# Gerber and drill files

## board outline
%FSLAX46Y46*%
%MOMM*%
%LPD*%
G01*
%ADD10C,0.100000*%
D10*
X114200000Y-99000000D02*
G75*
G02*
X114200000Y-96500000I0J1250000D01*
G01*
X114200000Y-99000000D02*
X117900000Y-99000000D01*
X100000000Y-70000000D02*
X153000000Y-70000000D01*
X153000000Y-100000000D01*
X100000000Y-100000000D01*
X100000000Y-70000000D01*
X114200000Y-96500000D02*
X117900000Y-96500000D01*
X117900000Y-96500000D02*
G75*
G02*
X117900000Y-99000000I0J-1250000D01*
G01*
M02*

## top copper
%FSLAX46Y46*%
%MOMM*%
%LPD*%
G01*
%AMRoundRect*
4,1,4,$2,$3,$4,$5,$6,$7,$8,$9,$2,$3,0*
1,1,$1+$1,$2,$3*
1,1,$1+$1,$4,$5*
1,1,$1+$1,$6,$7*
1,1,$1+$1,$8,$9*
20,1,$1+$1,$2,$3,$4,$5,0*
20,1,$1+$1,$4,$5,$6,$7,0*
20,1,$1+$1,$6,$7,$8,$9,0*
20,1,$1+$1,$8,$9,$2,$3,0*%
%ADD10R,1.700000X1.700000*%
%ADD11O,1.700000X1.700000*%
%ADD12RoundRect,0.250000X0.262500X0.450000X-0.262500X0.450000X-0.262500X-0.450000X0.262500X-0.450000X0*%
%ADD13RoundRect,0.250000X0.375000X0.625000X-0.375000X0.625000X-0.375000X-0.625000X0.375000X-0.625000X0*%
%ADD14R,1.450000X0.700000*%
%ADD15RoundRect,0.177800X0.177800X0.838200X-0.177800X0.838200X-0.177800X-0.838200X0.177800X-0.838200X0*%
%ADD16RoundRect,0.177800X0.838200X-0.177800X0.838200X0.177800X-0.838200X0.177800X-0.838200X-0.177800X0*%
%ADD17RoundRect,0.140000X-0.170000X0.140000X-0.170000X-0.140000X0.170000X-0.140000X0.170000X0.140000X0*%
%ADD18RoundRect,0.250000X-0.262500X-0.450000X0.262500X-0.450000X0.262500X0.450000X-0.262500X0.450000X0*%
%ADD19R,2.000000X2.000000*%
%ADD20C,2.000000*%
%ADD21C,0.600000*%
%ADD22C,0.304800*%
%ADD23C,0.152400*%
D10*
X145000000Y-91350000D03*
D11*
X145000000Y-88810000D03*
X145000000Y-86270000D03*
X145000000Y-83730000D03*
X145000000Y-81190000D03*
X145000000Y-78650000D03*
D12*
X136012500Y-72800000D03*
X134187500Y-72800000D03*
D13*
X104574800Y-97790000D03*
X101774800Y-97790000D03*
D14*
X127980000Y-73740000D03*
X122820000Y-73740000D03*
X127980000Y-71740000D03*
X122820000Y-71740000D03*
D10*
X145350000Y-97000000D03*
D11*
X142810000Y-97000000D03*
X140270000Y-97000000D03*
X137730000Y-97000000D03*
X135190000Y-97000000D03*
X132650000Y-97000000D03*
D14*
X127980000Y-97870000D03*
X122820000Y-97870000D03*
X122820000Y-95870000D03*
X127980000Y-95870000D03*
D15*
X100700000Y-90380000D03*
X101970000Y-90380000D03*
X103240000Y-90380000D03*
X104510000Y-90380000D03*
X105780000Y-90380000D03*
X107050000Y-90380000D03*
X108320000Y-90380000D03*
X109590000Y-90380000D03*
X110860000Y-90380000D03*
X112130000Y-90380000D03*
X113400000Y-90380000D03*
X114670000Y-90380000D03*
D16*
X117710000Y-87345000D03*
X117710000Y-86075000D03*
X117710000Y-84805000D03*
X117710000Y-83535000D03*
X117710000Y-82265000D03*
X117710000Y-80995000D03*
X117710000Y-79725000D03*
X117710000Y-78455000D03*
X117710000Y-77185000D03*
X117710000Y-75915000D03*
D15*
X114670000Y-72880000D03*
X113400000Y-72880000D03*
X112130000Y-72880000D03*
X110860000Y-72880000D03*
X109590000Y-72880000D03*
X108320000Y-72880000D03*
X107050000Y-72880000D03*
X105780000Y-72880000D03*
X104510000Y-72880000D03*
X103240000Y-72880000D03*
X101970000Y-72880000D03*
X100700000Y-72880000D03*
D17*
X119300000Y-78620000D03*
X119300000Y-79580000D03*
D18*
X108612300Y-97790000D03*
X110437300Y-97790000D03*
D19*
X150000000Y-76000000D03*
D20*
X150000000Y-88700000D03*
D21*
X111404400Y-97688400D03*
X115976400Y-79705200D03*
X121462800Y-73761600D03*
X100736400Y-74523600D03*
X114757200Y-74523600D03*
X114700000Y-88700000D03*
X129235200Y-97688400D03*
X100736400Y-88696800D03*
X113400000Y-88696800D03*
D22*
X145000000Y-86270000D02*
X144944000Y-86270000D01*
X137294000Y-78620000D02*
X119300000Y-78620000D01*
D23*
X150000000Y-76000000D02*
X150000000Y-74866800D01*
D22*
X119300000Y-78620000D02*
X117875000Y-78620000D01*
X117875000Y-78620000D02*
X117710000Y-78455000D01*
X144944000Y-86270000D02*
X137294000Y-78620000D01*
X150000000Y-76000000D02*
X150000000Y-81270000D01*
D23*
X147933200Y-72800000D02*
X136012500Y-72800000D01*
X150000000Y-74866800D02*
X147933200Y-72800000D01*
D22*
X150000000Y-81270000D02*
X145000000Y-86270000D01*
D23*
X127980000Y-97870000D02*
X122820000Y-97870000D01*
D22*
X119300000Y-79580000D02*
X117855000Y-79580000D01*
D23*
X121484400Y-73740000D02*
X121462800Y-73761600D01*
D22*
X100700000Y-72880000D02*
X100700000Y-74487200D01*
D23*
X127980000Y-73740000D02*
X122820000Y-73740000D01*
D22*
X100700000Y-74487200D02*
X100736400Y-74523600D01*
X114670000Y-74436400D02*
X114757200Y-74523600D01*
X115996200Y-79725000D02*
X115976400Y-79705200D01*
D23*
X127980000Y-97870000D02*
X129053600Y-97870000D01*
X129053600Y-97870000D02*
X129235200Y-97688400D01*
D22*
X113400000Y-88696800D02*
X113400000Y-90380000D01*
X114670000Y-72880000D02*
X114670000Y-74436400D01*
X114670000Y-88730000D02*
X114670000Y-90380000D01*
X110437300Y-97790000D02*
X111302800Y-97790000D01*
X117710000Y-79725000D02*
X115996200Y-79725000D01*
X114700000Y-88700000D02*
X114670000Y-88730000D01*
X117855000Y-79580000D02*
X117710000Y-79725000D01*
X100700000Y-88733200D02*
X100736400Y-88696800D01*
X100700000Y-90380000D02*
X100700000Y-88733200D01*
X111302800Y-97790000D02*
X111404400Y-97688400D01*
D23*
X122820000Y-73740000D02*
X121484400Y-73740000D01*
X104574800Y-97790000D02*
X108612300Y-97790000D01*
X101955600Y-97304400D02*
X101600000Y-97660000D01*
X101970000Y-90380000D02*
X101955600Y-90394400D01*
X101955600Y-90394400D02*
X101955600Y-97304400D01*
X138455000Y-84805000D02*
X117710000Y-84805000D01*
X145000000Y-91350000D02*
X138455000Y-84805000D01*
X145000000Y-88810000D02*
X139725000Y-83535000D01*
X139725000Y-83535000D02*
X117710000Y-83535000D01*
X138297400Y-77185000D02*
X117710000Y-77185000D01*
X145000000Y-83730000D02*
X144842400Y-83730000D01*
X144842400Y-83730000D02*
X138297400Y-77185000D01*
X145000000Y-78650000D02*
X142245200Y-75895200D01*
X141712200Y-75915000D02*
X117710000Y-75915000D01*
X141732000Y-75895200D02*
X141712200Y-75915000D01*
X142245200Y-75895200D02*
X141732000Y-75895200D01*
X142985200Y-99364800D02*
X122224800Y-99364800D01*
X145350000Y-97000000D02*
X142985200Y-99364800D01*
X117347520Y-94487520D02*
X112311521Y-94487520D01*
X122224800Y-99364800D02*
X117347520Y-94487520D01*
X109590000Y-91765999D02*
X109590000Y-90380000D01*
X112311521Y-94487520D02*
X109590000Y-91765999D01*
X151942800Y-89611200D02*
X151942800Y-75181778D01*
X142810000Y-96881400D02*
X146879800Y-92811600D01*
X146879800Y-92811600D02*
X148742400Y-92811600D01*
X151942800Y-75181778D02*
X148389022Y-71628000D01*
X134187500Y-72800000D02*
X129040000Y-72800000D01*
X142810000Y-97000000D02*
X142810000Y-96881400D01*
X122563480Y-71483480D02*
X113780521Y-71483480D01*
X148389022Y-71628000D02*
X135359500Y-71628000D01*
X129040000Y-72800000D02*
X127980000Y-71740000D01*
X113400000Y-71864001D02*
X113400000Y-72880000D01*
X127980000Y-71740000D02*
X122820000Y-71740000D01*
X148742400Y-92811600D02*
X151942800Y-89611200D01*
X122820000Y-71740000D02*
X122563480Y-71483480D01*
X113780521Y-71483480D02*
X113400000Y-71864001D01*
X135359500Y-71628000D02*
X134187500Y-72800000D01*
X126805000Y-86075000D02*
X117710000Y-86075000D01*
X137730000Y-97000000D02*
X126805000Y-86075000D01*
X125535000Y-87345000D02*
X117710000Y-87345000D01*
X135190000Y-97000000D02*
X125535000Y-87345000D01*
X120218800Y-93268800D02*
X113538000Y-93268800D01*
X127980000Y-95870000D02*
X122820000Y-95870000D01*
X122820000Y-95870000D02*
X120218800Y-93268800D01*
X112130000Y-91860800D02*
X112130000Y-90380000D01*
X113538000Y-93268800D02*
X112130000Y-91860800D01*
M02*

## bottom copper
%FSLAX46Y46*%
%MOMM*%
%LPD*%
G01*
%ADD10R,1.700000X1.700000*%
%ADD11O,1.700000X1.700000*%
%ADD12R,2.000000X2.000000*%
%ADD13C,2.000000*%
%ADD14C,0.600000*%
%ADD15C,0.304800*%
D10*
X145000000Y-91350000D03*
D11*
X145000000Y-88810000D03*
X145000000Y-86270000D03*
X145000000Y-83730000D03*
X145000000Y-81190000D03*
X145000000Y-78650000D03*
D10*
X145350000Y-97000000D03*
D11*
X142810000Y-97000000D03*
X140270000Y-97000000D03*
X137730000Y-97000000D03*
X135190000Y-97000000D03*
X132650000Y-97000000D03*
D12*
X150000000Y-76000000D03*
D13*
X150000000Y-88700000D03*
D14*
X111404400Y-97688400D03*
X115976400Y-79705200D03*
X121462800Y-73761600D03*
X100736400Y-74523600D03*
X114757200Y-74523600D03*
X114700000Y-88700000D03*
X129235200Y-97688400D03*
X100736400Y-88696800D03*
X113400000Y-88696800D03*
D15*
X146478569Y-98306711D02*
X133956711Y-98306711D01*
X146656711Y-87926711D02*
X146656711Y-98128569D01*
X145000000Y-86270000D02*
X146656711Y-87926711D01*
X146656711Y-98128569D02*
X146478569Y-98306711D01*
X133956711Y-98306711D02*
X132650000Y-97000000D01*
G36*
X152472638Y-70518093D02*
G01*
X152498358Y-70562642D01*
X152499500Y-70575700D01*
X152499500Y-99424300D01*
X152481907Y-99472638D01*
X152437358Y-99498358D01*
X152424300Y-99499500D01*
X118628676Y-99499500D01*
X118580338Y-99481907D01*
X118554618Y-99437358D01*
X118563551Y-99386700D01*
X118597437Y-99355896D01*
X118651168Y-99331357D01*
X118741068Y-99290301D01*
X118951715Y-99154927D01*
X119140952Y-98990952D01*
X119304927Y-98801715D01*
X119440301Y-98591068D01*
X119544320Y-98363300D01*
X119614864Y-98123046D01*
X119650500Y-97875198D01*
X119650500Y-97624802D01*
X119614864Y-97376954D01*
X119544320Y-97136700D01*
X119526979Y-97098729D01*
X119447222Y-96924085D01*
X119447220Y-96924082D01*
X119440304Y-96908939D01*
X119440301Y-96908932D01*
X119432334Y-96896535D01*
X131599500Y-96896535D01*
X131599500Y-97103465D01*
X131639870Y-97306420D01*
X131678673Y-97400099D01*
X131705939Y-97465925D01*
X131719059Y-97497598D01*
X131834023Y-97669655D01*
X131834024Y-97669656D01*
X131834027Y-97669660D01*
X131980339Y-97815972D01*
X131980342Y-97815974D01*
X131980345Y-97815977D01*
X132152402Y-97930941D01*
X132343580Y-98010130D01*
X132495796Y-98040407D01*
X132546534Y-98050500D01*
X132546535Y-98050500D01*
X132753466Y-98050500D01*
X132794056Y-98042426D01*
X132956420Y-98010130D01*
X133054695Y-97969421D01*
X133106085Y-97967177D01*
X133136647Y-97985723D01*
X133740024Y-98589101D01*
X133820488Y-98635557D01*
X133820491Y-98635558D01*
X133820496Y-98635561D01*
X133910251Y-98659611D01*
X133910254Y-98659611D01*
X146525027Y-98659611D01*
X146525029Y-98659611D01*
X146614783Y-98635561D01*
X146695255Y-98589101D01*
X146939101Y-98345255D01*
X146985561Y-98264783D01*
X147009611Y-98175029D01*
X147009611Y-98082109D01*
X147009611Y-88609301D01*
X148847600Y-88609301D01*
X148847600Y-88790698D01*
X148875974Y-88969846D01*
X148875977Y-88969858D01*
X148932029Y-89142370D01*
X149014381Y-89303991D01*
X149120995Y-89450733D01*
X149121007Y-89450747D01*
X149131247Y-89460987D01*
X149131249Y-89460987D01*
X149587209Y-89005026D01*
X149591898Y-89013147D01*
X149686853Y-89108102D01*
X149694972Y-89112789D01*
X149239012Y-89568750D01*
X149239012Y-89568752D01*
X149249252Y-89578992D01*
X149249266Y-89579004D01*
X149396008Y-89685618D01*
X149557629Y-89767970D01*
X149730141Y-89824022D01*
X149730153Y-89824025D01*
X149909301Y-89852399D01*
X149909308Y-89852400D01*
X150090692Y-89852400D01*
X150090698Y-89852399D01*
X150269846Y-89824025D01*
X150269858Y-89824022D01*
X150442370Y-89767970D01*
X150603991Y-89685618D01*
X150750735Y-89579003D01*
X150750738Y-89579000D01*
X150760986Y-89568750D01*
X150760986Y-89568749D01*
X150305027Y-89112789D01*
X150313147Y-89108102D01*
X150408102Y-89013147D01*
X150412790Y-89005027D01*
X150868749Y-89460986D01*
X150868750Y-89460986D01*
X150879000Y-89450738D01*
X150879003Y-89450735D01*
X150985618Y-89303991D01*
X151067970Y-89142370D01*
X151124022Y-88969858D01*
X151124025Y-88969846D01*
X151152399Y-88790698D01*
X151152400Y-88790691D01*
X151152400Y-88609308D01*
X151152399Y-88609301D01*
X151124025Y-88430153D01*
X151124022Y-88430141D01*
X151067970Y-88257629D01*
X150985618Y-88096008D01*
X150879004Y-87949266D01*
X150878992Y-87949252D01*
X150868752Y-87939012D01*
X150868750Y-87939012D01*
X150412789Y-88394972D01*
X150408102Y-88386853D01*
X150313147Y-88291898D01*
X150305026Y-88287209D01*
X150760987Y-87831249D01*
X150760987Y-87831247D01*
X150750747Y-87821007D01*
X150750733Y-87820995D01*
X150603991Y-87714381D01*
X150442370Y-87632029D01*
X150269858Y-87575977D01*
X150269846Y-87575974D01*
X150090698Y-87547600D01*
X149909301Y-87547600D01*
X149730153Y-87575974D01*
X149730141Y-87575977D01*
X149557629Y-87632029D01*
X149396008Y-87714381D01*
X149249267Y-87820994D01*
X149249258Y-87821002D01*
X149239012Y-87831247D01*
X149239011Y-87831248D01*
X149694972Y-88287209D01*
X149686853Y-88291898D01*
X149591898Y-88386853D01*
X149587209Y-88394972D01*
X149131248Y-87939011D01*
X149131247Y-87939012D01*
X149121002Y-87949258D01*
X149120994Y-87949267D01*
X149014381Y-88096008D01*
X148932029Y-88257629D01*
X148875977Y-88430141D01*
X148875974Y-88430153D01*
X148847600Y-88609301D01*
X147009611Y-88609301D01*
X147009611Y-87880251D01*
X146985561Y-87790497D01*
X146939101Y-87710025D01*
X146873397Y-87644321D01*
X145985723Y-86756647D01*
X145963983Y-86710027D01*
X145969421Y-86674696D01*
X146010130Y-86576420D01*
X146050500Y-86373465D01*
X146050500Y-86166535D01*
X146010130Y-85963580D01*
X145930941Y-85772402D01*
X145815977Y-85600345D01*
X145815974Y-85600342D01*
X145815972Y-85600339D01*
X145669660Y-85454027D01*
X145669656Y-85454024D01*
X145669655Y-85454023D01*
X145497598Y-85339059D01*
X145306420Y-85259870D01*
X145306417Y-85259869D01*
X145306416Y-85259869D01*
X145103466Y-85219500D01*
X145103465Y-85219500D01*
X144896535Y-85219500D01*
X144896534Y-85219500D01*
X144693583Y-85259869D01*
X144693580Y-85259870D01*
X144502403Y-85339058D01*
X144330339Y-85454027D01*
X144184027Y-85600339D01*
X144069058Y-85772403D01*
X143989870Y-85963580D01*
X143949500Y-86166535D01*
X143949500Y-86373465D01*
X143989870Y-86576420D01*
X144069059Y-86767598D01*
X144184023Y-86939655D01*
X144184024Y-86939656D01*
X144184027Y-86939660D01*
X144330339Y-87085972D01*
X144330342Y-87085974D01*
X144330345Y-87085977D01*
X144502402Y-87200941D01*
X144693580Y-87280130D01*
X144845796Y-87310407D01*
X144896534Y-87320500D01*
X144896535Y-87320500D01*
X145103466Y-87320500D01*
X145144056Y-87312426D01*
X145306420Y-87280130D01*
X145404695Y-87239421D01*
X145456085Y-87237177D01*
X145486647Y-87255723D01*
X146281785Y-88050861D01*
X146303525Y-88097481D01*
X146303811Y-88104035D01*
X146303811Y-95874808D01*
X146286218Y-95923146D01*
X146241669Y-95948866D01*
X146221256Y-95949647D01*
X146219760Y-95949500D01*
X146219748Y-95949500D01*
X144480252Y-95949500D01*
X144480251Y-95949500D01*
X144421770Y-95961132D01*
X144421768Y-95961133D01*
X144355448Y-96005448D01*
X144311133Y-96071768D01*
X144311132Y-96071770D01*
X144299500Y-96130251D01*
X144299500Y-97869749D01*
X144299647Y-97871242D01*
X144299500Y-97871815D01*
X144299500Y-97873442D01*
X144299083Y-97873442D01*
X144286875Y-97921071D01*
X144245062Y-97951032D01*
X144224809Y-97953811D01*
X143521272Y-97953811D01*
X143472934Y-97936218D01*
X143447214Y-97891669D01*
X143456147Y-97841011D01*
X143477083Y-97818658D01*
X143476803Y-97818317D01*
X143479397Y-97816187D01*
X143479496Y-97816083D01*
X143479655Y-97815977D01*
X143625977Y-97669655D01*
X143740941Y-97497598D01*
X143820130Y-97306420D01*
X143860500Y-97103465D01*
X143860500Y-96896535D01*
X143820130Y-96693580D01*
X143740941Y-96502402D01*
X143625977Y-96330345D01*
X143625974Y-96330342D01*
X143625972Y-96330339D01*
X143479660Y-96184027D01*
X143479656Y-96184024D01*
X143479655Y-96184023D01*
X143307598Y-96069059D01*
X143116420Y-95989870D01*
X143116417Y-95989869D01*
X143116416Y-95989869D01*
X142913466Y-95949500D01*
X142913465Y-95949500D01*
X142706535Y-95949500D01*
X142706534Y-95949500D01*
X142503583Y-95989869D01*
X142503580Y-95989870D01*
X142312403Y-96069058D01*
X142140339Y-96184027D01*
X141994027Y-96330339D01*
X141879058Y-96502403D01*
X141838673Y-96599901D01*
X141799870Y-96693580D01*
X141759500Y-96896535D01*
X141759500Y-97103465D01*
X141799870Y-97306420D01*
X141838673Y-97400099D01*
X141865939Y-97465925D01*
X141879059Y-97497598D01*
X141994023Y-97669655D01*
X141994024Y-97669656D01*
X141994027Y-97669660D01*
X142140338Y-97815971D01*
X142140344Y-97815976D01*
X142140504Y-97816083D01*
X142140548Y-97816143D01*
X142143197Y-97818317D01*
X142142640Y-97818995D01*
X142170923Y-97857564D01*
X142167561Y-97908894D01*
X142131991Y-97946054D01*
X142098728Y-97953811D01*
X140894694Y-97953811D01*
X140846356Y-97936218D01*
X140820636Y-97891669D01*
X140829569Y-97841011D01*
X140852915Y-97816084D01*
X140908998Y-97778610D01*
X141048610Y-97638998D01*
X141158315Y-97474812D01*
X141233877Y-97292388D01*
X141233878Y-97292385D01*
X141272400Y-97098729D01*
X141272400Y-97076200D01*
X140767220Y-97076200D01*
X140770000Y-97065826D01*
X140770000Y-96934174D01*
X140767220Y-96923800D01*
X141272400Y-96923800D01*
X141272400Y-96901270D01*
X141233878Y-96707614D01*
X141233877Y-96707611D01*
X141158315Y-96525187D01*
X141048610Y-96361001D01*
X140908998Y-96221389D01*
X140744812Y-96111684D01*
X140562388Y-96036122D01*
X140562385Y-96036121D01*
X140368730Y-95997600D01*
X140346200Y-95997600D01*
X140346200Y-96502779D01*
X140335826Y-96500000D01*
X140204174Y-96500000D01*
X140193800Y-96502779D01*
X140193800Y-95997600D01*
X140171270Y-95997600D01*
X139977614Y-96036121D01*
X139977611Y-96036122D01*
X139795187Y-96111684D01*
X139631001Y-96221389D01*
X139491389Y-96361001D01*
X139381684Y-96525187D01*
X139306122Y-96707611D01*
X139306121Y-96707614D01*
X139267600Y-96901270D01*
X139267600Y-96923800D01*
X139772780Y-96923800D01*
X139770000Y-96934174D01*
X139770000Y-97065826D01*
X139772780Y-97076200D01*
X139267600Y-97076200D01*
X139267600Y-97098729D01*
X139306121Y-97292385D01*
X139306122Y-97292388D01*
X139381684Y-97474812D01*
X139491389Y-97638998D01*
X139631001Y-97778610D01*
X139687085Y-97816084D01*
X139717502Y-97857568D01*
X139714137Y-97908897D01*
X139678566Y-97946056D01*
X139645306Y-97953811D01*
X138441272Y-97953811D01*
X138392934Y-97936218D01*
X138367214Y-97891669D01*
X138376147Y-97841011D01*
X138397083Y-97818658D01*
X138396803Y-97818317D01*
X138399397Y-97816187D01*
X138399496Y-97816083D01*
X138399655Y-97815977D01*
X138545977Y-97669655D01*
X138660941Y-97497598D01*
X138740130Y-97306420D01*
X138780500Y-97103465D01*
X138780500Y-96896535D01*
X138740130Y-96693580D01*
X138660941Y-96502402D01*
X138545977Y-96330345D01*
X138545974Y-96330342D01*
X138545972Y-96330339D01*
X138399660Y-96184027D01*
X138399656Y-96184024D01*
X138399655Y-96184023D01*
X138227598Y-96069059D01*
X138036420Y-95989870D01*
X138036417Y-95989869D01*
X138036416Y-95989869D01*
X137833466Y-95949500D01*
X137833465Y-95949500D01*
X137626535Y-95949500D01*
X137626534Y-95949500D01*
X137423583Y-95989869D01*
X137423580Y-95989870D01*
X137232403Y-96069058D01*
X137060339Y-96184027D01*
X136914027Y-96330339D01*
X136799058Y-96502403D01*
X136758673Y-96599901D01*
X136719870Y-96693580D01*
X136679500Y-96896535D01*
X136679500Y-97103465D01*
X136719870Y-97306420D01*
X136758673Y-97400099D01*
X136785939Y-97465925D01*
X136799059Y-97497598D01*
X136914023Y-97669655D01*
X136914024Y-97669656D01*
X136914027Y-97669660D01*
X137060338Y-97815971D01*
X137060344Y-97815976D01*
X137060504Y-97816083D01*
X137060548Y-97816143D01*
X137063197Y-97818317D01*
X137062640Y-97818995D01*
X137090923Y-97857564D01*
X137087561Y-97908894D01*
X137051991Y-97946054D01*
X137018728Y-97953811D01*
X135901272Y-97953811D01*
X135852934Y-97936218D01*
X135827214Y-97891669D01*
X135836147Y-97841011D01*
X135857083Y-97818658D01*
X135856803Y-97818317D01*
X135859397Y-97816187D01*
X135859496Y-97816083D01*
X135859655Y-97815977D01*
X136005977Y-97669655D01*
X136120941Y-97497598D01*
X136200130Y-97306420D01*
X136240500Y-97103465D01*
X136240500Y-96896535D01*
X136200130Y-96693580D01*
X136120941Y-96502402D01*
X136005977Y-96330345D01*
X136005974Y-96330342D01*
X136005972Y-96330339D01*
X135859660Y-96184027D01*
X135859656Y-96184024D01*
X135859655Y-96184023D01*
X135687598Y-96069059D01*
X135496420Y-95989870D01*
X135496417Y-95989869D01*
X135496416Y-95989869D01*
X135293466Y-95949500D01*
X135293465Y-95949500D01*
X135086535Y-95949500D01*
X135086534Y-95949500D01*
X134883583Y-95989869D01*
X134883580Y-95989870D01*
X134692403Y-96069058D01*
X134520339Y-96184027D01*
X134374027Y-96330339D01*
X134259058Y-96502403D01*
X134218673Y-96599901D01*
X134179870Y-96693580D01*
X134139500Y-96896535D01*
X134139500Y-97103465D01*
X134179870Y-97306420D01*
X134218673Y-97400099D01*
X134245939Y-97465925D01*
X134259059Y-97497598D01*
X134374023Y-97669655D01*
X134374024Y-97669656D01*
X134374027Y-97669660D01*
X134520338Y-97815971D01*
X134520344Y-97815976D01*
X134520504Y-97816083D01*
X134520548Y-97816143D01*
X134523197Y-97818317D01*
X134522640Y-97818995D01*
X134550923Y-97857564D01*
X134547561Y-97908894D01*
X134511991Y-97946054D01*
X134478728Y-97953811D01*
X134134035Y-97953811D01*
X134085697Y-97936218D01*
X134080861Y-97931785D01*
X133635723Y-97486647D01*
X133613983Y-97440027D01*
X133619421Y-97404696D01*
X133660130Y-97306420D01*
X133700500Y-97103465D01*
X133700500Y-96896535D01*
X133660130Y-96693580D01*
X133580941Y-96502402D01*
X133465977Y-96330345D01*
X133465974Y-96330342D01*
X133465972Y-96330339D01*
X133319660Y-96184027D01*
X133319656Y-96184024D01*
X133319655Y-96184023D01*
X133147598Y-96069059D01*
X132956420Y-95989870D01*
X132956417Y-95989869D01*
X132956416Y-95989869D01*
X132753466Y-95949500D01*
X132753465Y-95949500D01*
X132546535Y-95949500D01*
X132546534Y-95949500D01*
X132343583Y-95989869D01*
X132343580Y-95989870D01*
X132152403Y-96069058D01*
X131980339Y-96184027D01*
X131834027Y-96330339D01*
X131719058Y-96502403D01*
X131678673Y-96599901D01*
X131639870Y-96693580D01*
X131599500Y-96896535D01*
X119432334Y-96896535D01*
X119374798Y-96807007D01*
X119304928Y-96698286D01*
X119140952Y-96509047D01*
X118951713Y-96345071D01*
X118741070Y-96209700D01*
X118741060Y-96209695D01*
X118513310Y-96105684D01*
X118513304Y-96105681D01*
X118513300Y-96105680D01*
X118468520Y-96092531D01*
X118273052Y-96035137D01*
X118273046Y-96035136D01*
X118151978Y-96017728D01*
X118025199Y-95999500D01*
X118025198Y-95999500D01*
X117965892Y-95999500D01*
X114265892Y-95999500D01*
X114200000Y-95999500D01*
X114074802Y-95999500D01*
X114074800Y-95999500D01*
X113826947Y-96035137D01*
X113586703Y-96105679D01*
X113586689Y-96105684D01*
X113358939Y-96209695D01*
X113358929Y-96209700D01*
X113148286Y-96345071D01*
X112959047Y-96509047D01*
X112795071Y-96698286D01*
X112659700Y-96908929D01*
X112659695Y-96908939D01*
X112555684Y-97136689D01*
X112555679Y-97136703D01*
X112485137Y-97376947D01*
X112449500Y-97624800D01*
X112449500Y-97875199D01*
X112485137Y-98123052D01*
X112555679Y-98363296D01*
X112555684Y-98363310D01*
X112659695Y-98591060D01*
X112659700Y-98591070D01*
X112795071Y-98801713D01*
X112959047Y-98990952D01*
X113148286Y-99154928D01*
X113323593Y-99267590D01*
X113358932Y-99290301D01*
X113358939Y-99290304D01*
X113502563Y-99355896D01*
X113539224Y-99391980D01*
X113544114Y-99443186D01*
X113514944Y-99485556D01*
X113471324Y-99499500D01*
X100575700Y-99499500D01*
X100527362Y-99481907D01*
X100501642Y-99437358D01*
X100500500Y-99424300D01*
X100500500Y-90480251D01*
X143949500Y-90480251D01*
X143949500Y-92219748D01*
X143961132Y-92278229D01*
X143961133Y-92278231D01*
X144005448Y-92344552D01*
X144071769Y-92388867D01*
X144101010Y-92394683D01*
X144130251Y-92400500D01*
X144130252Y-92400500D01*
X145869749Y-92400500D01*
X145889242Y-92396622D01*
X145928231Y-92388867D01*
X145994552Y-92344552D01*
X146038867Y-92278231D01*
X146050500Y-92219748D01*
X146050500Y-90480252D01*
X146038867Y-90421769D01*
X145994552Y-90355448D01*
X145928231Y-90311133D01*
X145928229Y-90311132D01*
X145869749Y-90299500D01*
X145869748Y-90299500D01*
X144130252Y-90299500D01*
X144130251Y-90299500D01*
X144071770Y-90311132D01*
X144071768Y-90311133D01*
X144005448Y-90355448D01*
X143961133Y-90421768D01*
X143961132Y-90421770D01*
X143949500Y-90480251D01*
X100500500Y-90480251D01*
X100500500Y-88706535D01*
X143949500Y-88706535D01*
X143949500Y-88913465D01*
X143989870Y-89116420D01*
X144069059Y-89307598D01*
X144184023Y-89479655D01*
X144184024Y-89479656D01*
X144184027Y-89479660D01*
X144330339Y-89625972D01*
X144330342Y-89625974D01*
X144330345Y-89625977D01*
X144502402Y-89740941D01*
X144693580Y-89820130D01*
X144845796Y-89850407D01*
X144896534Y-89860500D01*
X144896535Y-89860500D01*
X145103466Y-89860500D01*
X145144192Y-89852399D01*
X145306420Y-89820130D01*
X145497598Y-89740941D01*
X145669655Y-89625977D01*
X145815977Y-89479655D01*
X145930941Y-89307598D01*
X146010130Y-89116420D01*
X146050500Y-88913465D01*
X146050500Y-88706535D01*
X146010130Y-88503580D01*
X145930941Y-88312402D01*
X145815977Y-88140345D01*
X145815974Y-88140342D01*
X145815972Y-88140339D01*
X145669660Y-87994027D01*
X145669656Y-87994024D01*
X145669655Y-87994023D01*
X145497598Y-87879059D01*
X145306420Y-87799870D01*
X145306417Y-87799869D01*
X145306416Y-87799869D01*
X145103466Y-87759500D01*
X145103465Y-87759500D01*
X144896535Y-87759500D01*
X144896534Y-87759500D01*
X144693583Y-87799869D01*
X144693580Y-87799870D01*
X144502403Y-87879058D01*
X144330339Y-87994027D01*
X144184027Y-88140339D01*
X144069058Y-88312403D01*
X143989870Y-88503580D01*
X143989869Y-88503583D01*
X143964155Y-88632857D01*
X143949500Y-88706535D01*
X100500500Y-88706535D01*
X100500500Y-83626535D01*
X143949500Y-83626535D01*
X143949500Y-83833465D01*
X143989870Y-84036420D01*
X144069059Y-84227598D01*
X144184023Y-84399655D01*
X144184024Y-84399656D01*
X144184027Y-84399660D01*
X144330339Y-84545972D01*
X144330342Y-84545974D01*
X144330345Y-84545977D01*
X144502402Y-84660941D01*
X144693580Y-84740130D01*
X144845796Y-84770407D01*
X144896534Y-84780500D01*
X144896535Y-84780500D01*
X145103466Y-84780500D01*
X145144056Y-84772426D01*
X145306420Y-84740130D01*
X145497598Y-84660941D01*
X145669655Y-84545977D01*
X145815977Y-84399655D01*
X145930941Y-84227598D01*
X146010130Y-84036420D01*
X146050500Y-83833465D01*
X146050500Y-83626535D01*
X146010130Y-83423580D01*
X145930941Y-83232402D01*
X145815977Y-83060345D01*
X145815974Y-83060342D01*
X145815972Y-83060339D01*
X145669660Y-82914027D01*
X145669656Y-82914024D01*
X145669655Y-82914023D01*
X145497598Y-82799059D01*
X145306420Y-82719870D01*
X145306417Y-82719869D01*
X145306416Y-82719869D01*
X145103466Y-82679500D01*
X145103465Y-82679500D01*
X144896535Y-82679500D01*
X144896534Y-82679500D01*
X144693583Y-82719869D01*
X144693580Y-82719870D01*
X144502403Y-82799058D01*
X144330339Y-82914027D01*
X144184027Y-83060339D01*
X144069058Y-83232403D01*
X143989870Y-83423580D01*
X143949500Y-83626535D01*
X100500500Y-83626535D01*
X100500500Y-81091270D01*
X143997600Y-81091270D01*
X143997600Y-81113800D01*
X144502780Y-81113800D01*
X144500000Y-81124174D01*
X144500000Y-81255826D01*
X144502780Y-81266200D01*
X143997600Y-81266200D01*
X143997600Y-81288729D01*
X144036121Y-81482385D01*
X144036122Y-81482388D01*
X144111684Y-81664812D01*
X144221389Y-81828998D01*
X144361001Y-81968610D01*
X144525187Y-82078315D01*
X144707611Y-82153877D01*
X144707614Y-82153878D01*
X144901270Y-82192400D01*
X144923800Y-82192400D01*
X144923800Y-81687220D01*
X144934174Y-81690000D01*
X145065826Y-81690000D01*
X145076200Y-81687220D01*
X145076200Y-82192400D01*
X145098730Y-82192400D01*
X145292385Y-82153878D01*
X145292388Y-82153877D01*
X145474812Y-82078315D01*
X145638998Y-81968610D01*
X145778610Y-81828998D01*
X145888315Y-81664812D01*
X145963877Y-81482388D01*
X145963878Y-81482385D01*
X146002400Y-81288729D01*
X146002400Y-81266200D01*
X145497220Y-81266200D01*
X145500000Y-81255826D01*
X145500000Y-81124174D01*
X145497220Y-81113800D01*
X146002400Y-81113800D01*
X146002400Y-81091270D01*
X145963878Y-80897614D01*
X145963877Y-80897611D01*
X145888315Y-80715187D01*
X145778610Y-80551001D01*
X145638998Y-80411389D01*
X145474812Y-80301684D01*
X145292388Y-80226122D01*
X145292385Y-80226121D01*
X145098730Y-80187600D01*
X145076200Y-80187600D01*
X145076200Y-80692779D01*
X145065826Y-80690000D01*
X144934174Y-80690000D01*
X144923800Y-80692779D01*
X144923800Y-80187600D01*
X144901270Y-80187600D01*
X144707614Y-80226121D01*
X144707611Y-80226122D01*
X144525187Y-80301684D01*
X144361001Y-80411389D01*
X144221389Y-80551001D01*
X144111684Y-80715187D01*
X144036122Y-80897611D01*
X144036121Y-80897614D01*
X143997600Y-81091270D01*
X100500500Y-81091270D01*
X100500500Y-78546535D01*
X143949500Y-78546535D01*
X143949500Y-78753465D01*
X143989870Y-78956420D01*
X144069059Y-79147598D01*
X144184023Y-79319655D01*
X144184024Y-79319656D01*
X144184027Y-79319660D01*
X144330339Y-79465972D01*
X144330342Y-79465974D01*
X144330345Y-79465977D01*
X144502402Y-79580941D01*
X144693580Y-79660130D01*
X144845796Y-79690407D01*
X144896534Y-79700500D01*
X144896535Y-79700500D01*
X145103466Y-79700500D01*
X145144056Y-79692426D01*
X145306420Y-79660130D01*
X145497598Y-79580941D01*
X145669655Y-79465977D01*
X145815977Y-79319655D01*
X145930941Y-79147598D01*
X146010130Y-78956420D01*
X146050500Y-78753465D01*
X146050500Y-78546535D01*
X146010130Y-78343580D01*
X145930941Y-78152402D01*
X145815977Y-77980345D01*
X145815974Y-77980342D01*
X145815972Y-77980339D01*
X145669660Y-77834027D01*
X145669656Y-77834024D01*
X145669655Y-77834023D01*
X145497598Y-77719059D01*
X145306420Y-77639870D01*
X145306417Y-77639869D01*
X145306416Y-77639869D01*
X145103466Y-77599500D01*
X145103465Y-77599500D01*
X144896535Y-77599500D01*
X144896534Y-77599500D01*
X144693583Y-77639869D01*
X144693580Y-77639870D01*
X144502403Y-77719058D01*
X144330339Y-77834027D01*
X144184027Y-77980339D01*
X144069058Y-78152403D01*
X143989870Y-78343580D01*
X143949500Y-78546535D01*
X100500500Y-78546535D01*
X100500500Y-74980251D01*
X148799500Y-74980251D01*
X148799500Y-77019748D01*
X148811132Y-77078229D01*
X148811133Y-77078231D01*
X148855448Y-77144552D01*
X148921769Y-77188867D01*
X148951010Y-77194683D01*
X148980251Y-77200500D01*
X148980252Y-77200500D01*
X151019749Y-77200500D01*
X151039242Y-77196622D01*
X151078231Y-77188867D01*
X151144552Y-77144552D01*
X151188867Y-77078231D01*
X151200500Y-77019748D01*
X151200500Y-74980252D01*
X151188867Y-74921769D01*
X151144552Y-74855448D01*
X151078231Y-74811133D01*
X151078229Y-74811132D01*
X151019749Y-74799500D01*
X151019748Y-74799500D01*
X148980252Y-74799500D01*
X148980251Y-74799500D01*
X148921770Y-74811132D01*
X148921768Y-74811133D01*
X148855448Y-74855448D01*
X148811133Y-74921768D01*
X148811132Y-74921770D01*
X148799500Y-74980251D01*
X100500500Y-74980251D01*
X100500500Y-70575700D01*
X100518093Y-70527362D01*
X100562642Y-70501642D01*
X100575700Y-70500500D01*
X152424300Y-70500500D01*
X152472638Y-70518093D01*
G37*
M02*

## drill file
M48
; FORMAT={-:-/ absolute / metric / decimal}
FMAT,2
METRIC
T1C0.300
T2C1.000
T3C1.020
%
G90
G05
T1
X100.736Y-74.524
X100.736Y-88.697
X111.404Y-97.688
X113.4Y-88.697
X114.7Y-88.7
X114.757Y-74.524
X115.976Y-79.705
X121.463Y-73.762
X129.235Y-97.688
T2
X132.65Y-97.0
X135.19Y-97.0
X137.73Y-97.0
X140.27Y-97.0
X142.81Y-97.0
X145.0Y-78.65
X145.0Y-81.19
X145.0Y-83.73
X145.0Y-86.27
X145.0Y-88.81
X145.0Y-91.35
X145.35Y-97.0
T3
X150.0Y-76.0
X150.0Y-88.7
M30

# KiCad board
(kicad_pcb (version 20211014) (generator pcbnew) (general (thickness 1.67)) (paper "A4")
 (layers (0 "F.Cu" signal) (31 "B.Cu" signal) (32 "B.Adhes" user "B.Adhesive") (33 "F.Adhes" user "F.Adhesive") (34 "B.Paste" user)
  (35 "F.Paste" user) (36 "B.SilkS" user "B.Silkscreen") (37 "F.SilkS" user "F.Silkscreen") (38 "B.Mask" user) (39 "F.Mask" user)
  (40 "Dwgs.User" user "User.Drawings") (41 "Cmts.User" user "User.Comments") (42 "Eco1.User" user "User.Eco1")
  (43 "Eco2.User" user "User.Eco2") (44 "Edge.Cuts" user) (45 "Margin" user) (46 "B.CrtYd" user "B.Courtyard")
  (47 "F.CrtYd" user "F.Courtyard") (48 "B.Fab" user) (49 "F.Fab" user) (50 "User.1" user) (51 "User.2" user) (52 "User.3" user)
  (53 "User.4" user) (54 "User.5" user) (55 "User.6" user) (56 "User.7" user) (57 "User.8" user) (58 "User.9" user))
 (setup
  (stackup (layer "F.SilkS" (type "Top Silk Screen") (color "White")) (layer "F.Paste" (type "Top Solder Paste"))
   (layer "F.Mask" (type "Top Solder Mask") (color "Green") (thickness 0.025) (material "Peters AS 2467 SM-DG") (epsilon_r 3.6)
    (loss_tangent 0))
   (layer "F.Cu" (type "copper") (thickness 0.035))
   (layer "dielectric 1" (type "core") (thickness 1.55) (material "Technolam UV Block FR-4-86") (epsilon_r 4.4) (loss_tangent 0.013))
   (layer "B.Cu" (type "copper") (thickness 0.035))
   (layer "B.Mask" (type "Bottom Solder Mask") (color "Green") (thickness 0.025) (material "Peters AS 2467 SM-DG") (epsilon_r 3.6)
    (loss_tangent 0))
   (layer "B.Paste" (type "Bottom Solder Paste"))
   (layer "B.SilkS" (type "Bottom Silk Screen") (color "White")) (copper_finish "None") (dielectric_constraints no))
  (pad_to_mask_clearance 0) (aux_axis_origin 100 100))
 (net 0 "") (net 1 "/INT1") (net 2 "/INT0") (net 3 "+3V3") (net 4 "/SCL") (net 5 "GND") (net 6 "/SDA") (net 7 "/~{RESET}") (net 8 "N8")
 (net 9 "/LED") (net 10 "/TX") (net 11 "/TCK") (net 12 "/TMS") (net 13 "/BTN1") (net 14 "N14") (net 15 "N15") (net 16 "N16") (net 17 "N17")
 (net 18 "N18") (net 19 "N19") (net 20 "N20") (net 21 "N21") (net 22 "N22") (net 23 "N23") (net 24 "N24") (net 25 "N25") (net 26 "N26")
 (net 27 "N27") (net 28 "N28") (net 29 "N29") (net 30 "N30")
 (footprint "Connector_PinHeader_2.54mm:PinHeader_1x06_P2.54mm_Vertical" (layer "F.Cu") (at 145 91.35 180)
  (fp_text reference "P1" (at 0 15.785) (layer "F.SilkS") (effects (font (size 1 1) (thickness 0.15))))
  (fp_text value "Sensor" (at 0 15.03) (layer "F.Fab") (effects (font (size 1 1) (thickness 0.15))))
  (pad "1" thru_hole rect locked (at 0 0 180) (size 1.7 1.7) (drill 1) (layers *.Cu *.Mask) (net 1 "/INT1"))
  (pad "2" thru_hole oval locked (at 0 2.54 180) (size 1.7 1.7) (drill 1) (layers *.Cu *.Mask) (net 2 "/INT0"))
  (pad "3" thru_hole oval locked (at 0 5.08 180) (size 1.7 1.7) (drill 1) (layers *.Cu *.Mask) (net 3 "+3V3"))
  (pad "4" thru_hole oval locked (at 0 7.62 180) (size 1.7 1.7) (drill 1) (layers *.Cu *.Mask) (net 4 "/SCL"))
  (pad "5" thru_hole oval locked (at 0 10.16 180) (size 1.7 1.7) (drill 1) (layers *.Cu *.Mask) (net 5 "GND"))
  (pad "6" thru_hole oval locked (at 0 12.7 180) (size 1.7 1.7) (drill 1) (layers *.Cu *.Mask) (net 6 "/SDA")))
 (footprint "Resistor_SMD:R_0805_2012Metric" (layer "F.Cu") (at 135.1 72.8 180)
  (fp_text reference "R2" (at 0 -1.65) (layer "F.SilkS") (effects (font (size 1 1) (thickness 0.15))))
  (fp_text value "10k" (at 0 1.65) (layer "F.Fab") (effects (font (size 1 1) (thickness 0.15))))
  (pad "1" smd roundrect locked (at -0.9125 0 180) (size 1.025 1.4) (layers "F.Cu" "F.Paste" "F.Mask") (roundrect_rratio 0.243902439)
   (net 3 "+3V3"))
  (pad "2" smd roundrect locked (at 0.9125 0 180) (size 1.025 1.4) (layers "F.Cu" "F.Paste" "F.Mask") (roundrect_rratio 0.243902439)
   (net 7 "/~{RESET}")))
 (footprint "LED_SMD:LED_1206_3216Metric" (layer "F.Cu") (at 103.1748 97.79 180)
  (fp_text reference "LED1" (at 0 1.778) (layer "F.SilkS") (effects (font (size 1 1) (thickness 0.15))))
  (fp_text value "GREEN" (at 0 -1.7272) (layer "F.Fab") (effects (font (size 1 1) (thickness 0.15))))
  (pad "1" smd roundrect locked (at -1.4 0 180) (size 1.25 1.75) (layers "F.Cu" "F.Paste" "F.Mask") (roundrect_rratio 0.2) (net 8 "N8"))
  (pad "2" smd roundrect locked (at 1.4 0 180) (size 1.25 1.75) (layers "F.Cu" "F.Paste" "F.Mask") (roundrect_rratio 0.2) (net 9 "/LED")))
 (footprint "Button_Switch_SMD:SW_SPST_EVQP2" (layer "F.Cu") (at 125.4 72.74 180)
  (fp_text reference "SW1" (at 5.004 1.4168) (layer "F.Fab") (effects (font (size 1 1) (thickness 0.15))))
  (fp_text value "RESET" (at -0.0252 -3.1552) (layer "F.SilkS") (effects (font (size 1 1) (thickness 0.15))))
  (pad "1" smd rect locked (at -2.58 -1 180) (size 1.45 0.7) (layers "F.Cu" "F.Paste" "F.Mask") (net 5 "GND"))
  (pad "1" smd rect locked (at 2.58 -1 180) (size 1.45 0.7) (layers "F.Cu" "F.Paste" "F.Mask") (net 5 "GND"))
  (pad "2" smd rect locked (at -2.58 1 180) (size 1.45 0.7) (layers "F.Cu" "F.Paste" "F.Mask") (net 7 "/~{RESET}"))
  (pad "2" smd rect locked (at 2.58 1 180) (size 1.45 0.7) (layers "F.Cu" "F.Paste" "F.Mask") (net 7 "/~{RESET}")))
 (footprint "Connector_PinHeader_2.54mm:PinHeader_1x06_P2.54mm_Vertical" (layer "F.Cu") (at 145.35 97 -90)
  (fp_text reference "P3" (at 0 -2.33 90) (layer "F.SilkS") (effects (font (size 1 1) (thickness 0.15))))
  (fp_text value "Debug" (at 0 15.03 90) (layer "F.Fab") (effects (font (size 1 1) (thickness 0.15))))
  (pad "1" thru_hole rect locked (at 0 0 270) (size 1.7 1.7) (drill 1) (layers *.Cu *.Mask) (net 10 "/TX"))
  (pad "2" thru_hole oval locked (at 0 2.54 270) (size 1.7 1.7) (drill 1) (layers *.Cu *.Mask) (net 7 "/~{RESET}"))
  (pad "3" thru_hole oval locked (at 0 5.08 270) (size 1.7 1.7) (drill 1) (layers *.Cu *.Mask) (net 5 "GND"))
  (pad "4" thru_hole oval locked (at 0 7.62 270) (size 1.7 1.7) (drill 1) (layers *.Cu *.Mask) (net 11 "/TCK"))
  (pad "5" thru_hole oval locked (at 0 10.16 270) (size 1.7 1.7) (drill 1) (layers *.Cu *.Mask) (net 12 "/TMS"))
  (pad "6" thru_hole oval locked (at 0 12.7 270) (size 1.7 1.7) (drill 1) (layers *.Cu *.Mask) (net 3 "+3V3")))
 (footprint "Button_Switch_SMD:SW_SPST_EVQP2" (layer "F.Cu") (at 125.4 96.87 180)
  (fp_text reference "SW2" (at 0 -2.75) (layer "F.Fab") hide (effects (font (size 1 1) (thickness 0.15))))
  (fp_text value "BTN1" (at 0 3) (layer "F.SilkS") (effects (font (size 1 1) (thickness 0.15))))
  (pad "1" smd rect locked (at -2.58 -1 180) (size 1.45 0.7) (layers "F.Cu" "F.Paste" "F.Mask") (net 5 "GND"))
  (pad "1" smd rect locked (at 2.58 -1 180) (size 1.45 0.7) (layers "F.Cu" "F.Paste" "F.Mask") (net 5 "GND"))
  (pad "2" smd rect locked (at 2.58 1 180) (size 1.45 0.7) (layers "F.Cu" "F.Paste" "F.Mask") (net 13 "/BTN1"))
  (pad "2" smd rect locked (at -2.58 1 180) (size 1.45 0.7) (layers "F.Cu" "F.Paste" "F.Mask") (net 13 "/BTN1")))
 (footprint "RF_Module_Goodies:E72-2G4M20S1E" (layer "F.Cu") (at 100.7 81.63 90)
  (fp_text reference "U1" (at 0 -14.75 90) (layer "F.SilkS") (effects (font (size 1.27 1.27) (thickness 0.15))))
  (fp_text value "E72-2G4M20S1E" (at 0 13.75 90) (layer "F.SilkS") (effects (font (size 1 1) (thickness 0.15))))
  (pad "1" smd roundrect (at -8.75 0 180) (size 0.7112 2.032) (layers "F.Cu" "F.Paste" "F.Mask") (roundrect_rratio 0.25) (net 5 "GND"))
  (pad "2" smd roundrect (at -8.75 1.27 180) (size 0.7112 2.032) (layers "F.Cu" "F.Paste" "F.Mask") (roundrect_rratio 0.25) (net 9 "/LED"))
  (pad "3" smd roundrect (at -8.75 2.54 180) (size 0.7112 2.032) (layers "F.Cu" "F.Paste" "F.Mask") (roundrect_rratio 0.25) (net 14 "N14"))
  (pad "4" smd roundrect (at -8.75 3.81 180) (size 0.7112 2.032) (layers "F.Cu" "F.Paste" "F.Mask") (roundrect_rratio 0.25) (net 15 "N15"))
  (pad "5" smd roundrect (at -8.75 5.08 180) (size 0.7112 2.032) (layers "F.Cu" "F.Paste" "F.Mask") (roundrect_rratio 0.25) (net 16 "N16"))
  (pad "6" smd roundrect (at -8.75 6.35 180) (size 0.7112 2.032) (layers "F.Cu" "F.Paste" "F.Mask") (roundrect_rratio 0.25) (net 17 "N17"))
  (pad "7" smd roundrect (at -8.75 7.62 180) (size 0.7112 2.032) (layers "F.Cu" "F.Paste" "F.Mask") (roundrect_rratio 0.25) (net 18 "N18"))
  (pad "8" smd roundrect (at -8.75 8.89 180) (size 0.7112 2.032) (layers "F.Cu" "F.Paste" "F.Mask") (roundrect_rratio 0.25) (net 10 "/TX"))
  (pad "9" smd roundrect (at -8.75 10.16 180) (size 0.7112 2.032) (layers "F.Cu" "F.Paste" "F.Mask") (roundrect_rratio 0.25) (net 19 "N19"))
  (pad "10" smd roundrect (at -8.75 11.43 180) (size 0.7112 2.032) (layers "F.Cu" "F.Paste" "F.Mask") (roundrect_rratio 0.25)
   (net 13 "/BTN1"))
  (pad "11" smd roundrect (at -8.75 12.7 180) (size 0.7112 2.032) (layers "F.Cu" "F.Paste" "F.Mask") (roundrect_rratio 0.25) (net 5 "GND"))
  (pad "12" smd roundrect (at -8.75 13.97 180) (size 0.7112 2.032) (layers "F.Cu" "F.Paste" "F.Mask") (roundrect_rratio 0.25) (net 5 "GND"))
  (pad "13" smd roundrect (at -5.715 17.01 90) (size 0.7112 2.032) (layers "F.Cu" "F.Paste" "F.Mask") (roundrect_rratio 0.25)
   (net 12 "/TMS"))
  (pad "14" smd roundrect (at -4.445 17.01 90) (size 0.7112 2.032) (layers "F.Cu" "F.Paste" "F.Mask") (roundrect_rratio 0.25)
   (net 11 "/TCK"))
  (pad "15" smd roundrect (at -3.175 17.01 90) (size 0.7112 2.032) (layers "F.Cu" "F.Paste" "F.Mask") (roundrect_rratio 0.25)
   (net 1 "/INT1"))
  (pad "16" smd roundrect (at -1.905 17.01 90) (size 0.7112 2.032) (layers "F.Cu" "F.Paste" "F.Mask") (roundrect_rratio 0.25)
   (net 2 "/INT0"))
  (pad "17" smd roundrect (at -0.635 17.01 90) (size 0.7112 2.032) (layers "F.Cu" "F.Paste" "F.Mask") (roundrect_rratio 0.25) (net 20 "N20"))
  (pad "18" smd roundrect (at 0.635 17.01 90) (size 0.7112 2.032) (layers "F.Cu" "F.Paste" "F.Mask") (roundrect_rratio 0.25) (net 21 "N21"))
  (pad "19" smd roundrect (at 1.905 17.01 90) (size 0.7112 2.032) (layers "F.Cu" "F.Paste" "F.Mask") (roundrect_rratio 0.25) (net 5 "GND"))
  (pad "20" smd roundrect (at 3.175 17.01 90) (size 0.7112 2.032) (layers "F.Cu" "F.Paste" "F.Mask") (roundrect_rratio 0.25) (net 3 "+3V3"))
  (pad "21" smd roundrect (at 4.445 17.01 90) (size 0.7112 2.032) (layers "F.Cu" "F.Paste" "F.Mask") (roundrect_rratio 0.25) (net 4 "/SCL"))
  (pad "22" smd roundrect (at 5.715 17.01 90) (size 0.7112 2.032) (layers "F.Cu" "F.Paste" "F.Mask") (roundrect_rratio 0.25) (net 6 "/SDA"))
  (pad "23" smd roundrect (at 8.75 13.97 180) (size 0.7112 2.032) (layers "F.Cu" "F.Paste" "F.Mask") (roundrect_rratio 0.25) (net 5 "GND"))
  (pad "24" smd roundrect (at 8.75 12.7 180) (size 0.7112 2.032) (layers "F.Cu" "F.Paste" "F.Mask") (roundrect_rratio 0.25)
   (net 7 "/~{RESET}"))
  (pad "25" smd roundrect (at 8.75 11.43 180) (size 0.7112 2.032) (layers "F.Cu" "F.Paste" "F.Mask") (roundrect_rratio 0.25) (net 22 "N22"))
  (pad "26" smd roundrect (at 8.75 10.16 180) (size 0.7112 2.032) (layers "F.Cu" "F.Paste" "F.Mask") (roundrect_rratio 0.25) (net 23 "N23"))
  (pad "27" smd roundrect (at 8.75 8.89 180) (size 0.7112 2.032) (layers "F.Cu" "F.Paste" "F.Mask") (roundrect_rratio 0.25) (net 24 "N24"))
  (pad "28" smd roundrect (at 8.75 7.62 180) (size 0.7112 2.032) (layers "F.Cu" "F.Paste" "F.Mask") (roundrect_rratio 0.25) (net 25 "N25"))
  (pad "29" smd roundrect (at 8.75 6.35 180) (size 0.7112 2.032) (layers "F.Cu" "F.Paste" "F.Mask") (roundrect_rratio 0.25) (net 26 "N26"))
  (pad "30" smd roundrect (at 8.75 5.08 180) (size 0.7112 2.032) (layers "F.Cu" "F.Paste" "F.Mask") (roundrect_rratio 0.25) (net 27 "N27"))
  (pad "31" smd roundrect (at 8.75 3.81 180) (size 0.7112 2.032) (layers "F.Cu" "F.Paste" "F.Mask") (roundrect_rratio 0.25) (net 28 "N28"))
  (pad "32" smd roundrect (at 8.75 2.54 180) (size 0.7112 2.032) (layers "F.Cu" "F.Paste" "F.Mask") (roundrect_rratio 0.25) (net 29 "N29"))
  (pad "33" smd roundrect (at 8.75 1.27 180) (size 0.7112 2.032) (layers "F.Cu" "F.Paste" "F.Mask") (roundrect_rratio 0.25) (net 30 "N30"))
  (pad "34" smd roundrect (at 8.75 0 180) (size 0.7112 2.032) (layers "F.Cu" "F.Paste" "F.Mask") (roundrect_rratio 0.25) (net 5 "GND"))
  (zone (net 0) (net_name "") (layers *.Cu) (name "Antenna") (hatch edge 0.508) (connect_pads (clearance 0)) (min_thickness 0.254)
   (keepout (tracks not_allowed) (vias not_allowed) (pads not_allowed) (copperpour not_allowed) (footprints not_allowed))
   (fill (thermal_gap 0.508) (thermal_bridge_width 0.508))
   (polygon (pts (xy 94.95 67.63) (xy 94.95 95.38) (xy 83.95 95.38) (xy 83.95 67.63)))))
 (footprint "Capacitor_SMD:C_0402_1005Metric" (layer "F.Cu") (at 119.3 79.1 -90)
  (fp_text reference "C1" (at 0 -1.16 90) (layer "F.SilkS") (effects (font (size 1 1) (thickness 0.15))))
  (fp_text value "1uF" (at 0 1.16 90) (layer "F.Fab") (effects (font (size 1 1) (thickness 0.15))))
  (pad "1" smd roundrect locked (at -0.48 0 270) (size 0.56 0.62) (layers "F.Cu" "F.Paste" "F.Mask") (roundrect_rratio 0.25) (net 3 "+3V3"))
  (pad "2" smd roundrect locked (at 0.48 0 270) (size 0.56 0.62) (layers "F.Cu" "F.Paste" "F.Mask") (roundrect_rratio 0.25) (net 5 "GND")))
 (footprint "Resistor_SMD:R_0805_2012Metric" (layer "F.Cu") (at 109.5248 97.79)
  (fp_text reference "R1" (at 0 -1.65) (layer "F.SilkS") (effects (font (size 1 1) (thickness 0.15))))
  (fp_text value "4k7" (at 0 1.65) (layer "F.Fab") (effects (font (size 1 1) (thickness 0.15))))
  (pad "1" smd roundrect locked (at -0.9125 0) (size 1.025 1.4) (layers "F.Cu" "F.Paste" "F.Mask") (roundrect_rratio 0.243902439)
   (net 8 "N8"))
  (pad "2" smd roundrect locked (at 0.9125 0) (size 1.025 1.4) (layers "F.Cu" "F.Paste" "F.Mask") (roundrect_rratio 0.243902439)
   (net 5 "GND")))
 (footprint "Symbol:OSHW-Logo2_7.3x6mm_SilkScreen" (layer "B.Cu") (at 149.2 96.5 180)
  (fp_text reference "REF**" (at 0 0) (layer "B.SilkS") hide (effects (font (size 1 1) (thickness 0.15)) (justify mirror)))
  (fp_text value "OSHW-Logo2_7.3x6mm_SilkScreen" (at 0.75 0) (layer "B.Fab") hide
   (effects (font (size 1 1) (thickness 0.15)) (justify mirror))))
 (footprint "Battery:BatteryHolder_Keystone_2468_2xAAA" (layer "B.Cu") (at 150 76 180)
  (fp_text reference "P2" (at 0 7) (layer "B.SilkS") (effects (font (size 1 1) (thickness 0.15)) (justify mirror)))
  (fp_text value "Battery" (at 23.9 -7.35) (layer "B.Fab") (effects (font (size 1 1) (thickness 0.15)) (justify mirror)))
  (pad "1" thru_hole rect (at 0 0 180) (size 2 2) (drill 1.02) (layers *.Cu *.Mask) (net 3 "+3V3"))
  (pad "2" thru_hole circle (at 0 -12.7 180) (size 2 2) (drill 1.02) (layers *.Cu *.Mask) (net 5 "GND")))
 (gr_arc (start 114.2 99) (mid 112.95 97.75) (end 114.2 96.5) (layer "Edge.Cuts") (width 0.1))
 (gr_line (start 114.2 99) (end 117.9 99) (layer "Edge.Cuts") (width 0.1))
 (gr_rect (start 100 100) (end 153 70) (layer "Edge.Cuts") (width 0.1) (fill none))
 (gr_line (start 114.2 96.5) (end 117.9 96.5) (layer "Edge.Cuts") (width 0.1))
 (gr_arc (start 117.9 96.5) (mid 119.15 97.75) (end 117.9 99) (layer "Edge.Cuts") (width 0.1))
 (segment (start 145 86.27) (end 144.944 86.27) (width 0.3048) (layer "F.Cu") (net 3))
 (segment (start 137.294 78.62) (end 119.3 78.62) (width 0.3048) (layer "F.Cu") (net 3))
 (segment (start 150 76) (end 150 74.8668) (width 0.1524) (layer "F.Cu") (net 3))
 (segment (start 119.3 78.62) (end 117.875 78.62) (width 0.3048) (layer "F.Cu") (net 3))
 (segment (start 117.875 78.62) (end 117.71 78.455) (width 0.3048) (layer "F.Cu") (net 3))
 (segment (start 144.944 86.27) (end 137.294 78.62) (width 0.3048) (layer "F.Cu") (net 3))
 (segment (start 150 76) (end 150 81.27) (width 0.3048) (layer "F.Cu") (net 3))
 (segment (start 147.9332 72.8) (end 136.0125 72.8) (width 0.1524) (layer "F.Cu") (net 3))
 (segment (start 150 74.8668) (end 147.9332 72.8) (width 0.1524) (layer "F.Cu") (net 3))
 (segment (start 150 81.27) (end 145 86.27) (width 0.3048) (layer "F.Cu") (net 3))
 (segment (start 146.478569 98.306711) (end 133.956711 98.306711) (width 0.3048) (layer "B.Cu") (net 3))
 (segment (start 146.656711 87.926711) (end 146.656711 98.128569) (width 0.3048) (layer "B.Cu") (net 3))
 (segment (start 145 86.27) (end 146.656711 87.926711) (width 0.3048) (layer "B.Cu") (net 3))
 (segment (start 146.656711 98.128569) (end 146.478569 98.306711) (width 0.3048) (layer "B.Cu") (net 3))
 (segment (start 133.956711 98.306711) (end 132.65 97) (width 0.3048) (layer "B.Cu") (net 3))
 (segment (start 127.98 97.87) (end 122.82 97.87) (width 0.1524) (layer "F.Cu") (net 5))
 (segment (start 119.3 79.58) (end 117.855 79.58) (width 0.3048) (layer "F.Cu") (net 5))
 (segment (start 121.4844 73.74) (end 121.4628 73.7616) (width 0.1524) (layer "F.Cu") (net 5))
 (segment (start 100.7 72.88) (end 100.7 74.4872) (width 0.3048) (layer "F.Cu") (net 5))
 (segment (start 127.98 73.74) (end 122.82 73.74) (width 0.1524) (layer "F.Cu") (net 5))
 (segment (start 100.7 74.4872) (end 100.7364 74.5236) (width 0.3048) (layer "F.Cu") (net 5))
 (segment (start 114.67 74.4364) (end 114.7572 74.5236) (width 0.3048) (layer "F.Cu") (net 5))
 (segment (start 115.9962 79.725) (end 115.9764 79.7052) (width 0.3048) (layer "F.Cu") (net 5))
 (segment (start 127.98 97.87) (end 129.0536 97.87) (width 0.1524) (layer "F.Cu") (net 5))
 (segment (start 129.0536 97.87) (end 129.2352 97.6884) (width 0.1524) (layer "F.Cu") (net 5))
 (segment (start 113.4 88.6968) (end 113.4 90.38) (width 0.3048) (layer "F.Cu") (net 5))
 (segment (start 114.67 72.88) (end 114.67 74.4364) (width 0.3048) (layer "F.Cu") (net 5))
 (segment (start 114.67 88.73) (end 114.67 90.38) (width 0.3048) (layer "F.Cu") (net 5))
 (segment (start 110.4373 97.79) (end 111.3028 97.79) (width 0.3048) (layer "F.Cu") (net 5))
 (segment (start 117.71 79.725) (end 115.9962 79.725) (width 0.3048) (layer "F.Cu") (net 5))
 (segment (start 114.7 88.7) (end 114.67 88.73) (width 0.3048) (layer "F.Cu") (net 5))
 (segment (start 117.855 79.58) (end 117.71 79.725) (width 0.3048) (layer "F.Cu") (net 5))
 (segment (start 100.7 88.7332) (end 100.7364 88.6968) (width 0.3048) (layer "F.Cu") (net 5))
 (segment (start 100.7 90.38) (end 100.7 88.7332) (width 0.3048) (layer "F.Cu") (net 5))
 (segment (start 111.3028 97.79) (end 111.4044 97.6884) (width 0.3048) (layer "F.Cu") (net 5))
 (segment (start 122.82 73.74) (end 121.4844 73.74) (width 0.1524) (layer "F.Cu") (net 5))
 (via (at 111.4044 97.6884) (size 0.6) (drill 0.3) (layers "F.Cu" "B.Cu") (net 5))
 (via (at 115.9764 79.7052) (size 0.6) (drill 0.3) (layers "F.Cu" "B.Cu") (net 5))
 (via (at 121.4628 73.7616) (size 0.6) (drill 0.3) (layers "F.Cu" "B.Cu") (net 5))
 (via (at 100.7364 74.5236) (size 0.6) (drill 0.3) (layers "F.Cu" "B.Cu") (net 5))
 (via (at 114.7572 74.5236) (size 0.6) (drill 0.3) (layers "F.Cu" "B.Cu") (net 5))
 (via (at 114.7 88.7) (size 0.6) (drill 0.3) (layers "F.Cu" "B.Cu") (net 5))
 (via (at 129.2352 97.6884) (size 0.6) (drill 0.3) (layers "F.Cu" "B.Cu") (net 5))
 (via (at 100.7364 88.6968) (size 0.6) (drill 0.3) (layers "F.Cu" "B.Cu") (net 5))
 (via (at 113.4 88.6968) (size 0.6) (drill 0.3) (layers "F.Cu" "B.Cu") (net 5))
 (segment (start 104.5748 97.79) (end 108.6123 97.79) (width 0.1524) (layer "F.Cu") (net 8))
 (segment (start 101.9556 97.3044) (end 101.6 97.66) (width 0.1524) (layer "F.Cu") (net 9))
 (segment (start 101.97 90.38) (end 101.9556 90.3944) (width 0.1524) (layer "F.Cu") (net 9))
 (segment (start 101.9556 90.3944) (end 101.9556 97.3044) (width 0.1524) (layer "F.Cu") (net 9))
 (segment (start 138.455 84.805) (end 117.71 84.805) (width 0.1524) (layer "F.Cu") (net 1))
 (segment (start 145 91.35) (end 138.455 84.805) (width 0.1524) (layer "F.Cu") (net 1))
 (segment (start 145 88.81) (end 139.725 83.535) (width 0.1524) (layer "F.Cu") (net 2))
 (segment (start 139.725 83.535) (end 117.71 83.535) (width 0.1524) (layer "F.Cu") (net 2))
 (segment (start 138.2974 77.185) (end 117.71 77.185) (width 0.1524) (layer "F.Cu") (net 4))
 (segment (start 145 83.73) (end 144.8424 83.73) (width 0.1524) (layer "F.Cu") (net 4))
 (segment (start 144.8424 83.73) (end 138.2974 77.185) (width 0.1524) (layer "F.Cu") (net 4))
 (segment (start 145 78.65) (end 142.2452 75.8952) (width 0.1524) (layer "F.Cu") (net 6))
 (segment (start 141.7122 75.915) (end 117.71 75.915) (width 0.1524) (layer "F.Cu") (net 6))
 (segment (start 141.732 75.8952) (end 141.7122 75.915) (width 0.1524) (layer "F.Cu") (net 6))
 (segment (start 142.2452 75.8952) (end 141.732 75.8952) (width 0.1524) (layer "F.Cu") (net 6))
 (segment (start 142.9852 99.3648) (end 122.2248 99.3648) (width 0.1524) (layer "F.Cu") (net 10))
 (segment (start 145.35 97) (end 142.9852 99.3648) (width 0.1524) (layer "F.Cu") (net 10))
 (segment (start 117.34752 94.48752) (end 112.311521 94.48752) (width 0.1524) (layer "F.Cu") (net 10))
 (segment (start 122.2248 99.3648) (end 117.34752 94.48752) (width 0.1524) (layer "F.Cu") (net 10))
 (segment (start 109.59 91.765999) (end 109.59 90.38) (width 0.1524) (layer "F.Cu") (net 10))
 (segment (start 112.311521 94.48752) (end 109.59 91.765999) (width 0.1524) (layer "F.Cu") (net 10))
 (segment (start 151.9428 89.6112) (end 151.9428 75.181778) (width 0.1524) (layer "F.Cu") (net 7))
 (segment (start 142.81 96.8814) (end 146.8798 92.8116) (width 0.1524) (layer "F.Cu") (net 7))
 (segment (start 146.8798 92.8116) (end 148.7424 92.8116) (width 0.1524) (layer "F.Cu") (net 7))
 (segment (start 151.9428 75.181778) (end 148.389022 71.628) (width 0.1524) (layer "F.Cu") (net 7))
 (segment (start 134.1875 72.8) (end 129.04 72.8) (width 0.1524) (layer "F.Cu") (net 7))
 (segment (start 142.81 97) (end 142.81 96.8814) (width 0.1524) (layer "F.Cu") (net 7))
 (segment (start 122.56348 71.48348) (end 113.780521 71.48348) (width 0.1524) (layer "F.Cu") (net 7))
 (segment (start 148.389022 71.628) (end 135.3595 71.628) (width 0.1524) (layer "F.Cu") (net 7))
 (segment (start 129.04 72.8) (end 127.98 71.74) (width 0.1524) (layer "F.Cu") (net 7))
 (segment (start 113.4 71.864001) (end 113.4 72.88) (width 0.1524) (layer "F.Cu") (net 7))
 (segment (start 127.98 71.74) (end 122.82 71.74) (width 0.1524) (layer "F.Cu") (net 7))
 (segment (start 148.7424 92.8116) (end 151.9428 89.6112) (width 0.1524) (layer "F.Cu") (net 7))
 (segment (start 122.82 71.74) (end 122.56348 71.48348) (width 0.1524) (layer "F.Cu") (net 7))
 (segment (start 113.780521 71.48348) (end 113.4 71.864001) (width 0.1524) (layer "F.Cu") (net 7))
 (segment (start 135.3595 71.628) (end 134.1875 72.8) (width 0.1524) (layer "F.Cu") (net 7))
 (segment (start 126.805 86.075) (end 117.71 86.075) (width 0.1524) (layer "F.Cu") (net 11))
 (segment (start 137.73 97) (end 126.805 86.075) (width 0.1524) (layer "F.Cu") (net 11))
 (segment (start 125.535 87.345) (end 117.71 87.345) (width 0.1524) (layer "F.Cu") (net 12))
 (segment (start 135.19 97) (end 125.535 87.345) (width 0.1524) (layer "F.Cu") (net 12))
 (segment (start 120.2188 93.2688) (end 113.538 93.2688) (width 0.1524) (layer "F.Cu") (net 13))
 (segment (start 127.98 95.87) (end 122.82 95.87) (width 0.1524) (layer "F.Cu") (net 13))
 (segment (start 122.82 95.87) (end 120.2188 93.2688) (width 0.1524) (layer "F.Cu") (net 13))
 (segment (start 112.13 91.8608) (end 112.13 90.38) (width 0.1524) (layer "F.Cu") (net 13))
 (segment (start 113.538 93.2688) (end 112.13 91.8608) (width 0.1524) (layer "F.Cu") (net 13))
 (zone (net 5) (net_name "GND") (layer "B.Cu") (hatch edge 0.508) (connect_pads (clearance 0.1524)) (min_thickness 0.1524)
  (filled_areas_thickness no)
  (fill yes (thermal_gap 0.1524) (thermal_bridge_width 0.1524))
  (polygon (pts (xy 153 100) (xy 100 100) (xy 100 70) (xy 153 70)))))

